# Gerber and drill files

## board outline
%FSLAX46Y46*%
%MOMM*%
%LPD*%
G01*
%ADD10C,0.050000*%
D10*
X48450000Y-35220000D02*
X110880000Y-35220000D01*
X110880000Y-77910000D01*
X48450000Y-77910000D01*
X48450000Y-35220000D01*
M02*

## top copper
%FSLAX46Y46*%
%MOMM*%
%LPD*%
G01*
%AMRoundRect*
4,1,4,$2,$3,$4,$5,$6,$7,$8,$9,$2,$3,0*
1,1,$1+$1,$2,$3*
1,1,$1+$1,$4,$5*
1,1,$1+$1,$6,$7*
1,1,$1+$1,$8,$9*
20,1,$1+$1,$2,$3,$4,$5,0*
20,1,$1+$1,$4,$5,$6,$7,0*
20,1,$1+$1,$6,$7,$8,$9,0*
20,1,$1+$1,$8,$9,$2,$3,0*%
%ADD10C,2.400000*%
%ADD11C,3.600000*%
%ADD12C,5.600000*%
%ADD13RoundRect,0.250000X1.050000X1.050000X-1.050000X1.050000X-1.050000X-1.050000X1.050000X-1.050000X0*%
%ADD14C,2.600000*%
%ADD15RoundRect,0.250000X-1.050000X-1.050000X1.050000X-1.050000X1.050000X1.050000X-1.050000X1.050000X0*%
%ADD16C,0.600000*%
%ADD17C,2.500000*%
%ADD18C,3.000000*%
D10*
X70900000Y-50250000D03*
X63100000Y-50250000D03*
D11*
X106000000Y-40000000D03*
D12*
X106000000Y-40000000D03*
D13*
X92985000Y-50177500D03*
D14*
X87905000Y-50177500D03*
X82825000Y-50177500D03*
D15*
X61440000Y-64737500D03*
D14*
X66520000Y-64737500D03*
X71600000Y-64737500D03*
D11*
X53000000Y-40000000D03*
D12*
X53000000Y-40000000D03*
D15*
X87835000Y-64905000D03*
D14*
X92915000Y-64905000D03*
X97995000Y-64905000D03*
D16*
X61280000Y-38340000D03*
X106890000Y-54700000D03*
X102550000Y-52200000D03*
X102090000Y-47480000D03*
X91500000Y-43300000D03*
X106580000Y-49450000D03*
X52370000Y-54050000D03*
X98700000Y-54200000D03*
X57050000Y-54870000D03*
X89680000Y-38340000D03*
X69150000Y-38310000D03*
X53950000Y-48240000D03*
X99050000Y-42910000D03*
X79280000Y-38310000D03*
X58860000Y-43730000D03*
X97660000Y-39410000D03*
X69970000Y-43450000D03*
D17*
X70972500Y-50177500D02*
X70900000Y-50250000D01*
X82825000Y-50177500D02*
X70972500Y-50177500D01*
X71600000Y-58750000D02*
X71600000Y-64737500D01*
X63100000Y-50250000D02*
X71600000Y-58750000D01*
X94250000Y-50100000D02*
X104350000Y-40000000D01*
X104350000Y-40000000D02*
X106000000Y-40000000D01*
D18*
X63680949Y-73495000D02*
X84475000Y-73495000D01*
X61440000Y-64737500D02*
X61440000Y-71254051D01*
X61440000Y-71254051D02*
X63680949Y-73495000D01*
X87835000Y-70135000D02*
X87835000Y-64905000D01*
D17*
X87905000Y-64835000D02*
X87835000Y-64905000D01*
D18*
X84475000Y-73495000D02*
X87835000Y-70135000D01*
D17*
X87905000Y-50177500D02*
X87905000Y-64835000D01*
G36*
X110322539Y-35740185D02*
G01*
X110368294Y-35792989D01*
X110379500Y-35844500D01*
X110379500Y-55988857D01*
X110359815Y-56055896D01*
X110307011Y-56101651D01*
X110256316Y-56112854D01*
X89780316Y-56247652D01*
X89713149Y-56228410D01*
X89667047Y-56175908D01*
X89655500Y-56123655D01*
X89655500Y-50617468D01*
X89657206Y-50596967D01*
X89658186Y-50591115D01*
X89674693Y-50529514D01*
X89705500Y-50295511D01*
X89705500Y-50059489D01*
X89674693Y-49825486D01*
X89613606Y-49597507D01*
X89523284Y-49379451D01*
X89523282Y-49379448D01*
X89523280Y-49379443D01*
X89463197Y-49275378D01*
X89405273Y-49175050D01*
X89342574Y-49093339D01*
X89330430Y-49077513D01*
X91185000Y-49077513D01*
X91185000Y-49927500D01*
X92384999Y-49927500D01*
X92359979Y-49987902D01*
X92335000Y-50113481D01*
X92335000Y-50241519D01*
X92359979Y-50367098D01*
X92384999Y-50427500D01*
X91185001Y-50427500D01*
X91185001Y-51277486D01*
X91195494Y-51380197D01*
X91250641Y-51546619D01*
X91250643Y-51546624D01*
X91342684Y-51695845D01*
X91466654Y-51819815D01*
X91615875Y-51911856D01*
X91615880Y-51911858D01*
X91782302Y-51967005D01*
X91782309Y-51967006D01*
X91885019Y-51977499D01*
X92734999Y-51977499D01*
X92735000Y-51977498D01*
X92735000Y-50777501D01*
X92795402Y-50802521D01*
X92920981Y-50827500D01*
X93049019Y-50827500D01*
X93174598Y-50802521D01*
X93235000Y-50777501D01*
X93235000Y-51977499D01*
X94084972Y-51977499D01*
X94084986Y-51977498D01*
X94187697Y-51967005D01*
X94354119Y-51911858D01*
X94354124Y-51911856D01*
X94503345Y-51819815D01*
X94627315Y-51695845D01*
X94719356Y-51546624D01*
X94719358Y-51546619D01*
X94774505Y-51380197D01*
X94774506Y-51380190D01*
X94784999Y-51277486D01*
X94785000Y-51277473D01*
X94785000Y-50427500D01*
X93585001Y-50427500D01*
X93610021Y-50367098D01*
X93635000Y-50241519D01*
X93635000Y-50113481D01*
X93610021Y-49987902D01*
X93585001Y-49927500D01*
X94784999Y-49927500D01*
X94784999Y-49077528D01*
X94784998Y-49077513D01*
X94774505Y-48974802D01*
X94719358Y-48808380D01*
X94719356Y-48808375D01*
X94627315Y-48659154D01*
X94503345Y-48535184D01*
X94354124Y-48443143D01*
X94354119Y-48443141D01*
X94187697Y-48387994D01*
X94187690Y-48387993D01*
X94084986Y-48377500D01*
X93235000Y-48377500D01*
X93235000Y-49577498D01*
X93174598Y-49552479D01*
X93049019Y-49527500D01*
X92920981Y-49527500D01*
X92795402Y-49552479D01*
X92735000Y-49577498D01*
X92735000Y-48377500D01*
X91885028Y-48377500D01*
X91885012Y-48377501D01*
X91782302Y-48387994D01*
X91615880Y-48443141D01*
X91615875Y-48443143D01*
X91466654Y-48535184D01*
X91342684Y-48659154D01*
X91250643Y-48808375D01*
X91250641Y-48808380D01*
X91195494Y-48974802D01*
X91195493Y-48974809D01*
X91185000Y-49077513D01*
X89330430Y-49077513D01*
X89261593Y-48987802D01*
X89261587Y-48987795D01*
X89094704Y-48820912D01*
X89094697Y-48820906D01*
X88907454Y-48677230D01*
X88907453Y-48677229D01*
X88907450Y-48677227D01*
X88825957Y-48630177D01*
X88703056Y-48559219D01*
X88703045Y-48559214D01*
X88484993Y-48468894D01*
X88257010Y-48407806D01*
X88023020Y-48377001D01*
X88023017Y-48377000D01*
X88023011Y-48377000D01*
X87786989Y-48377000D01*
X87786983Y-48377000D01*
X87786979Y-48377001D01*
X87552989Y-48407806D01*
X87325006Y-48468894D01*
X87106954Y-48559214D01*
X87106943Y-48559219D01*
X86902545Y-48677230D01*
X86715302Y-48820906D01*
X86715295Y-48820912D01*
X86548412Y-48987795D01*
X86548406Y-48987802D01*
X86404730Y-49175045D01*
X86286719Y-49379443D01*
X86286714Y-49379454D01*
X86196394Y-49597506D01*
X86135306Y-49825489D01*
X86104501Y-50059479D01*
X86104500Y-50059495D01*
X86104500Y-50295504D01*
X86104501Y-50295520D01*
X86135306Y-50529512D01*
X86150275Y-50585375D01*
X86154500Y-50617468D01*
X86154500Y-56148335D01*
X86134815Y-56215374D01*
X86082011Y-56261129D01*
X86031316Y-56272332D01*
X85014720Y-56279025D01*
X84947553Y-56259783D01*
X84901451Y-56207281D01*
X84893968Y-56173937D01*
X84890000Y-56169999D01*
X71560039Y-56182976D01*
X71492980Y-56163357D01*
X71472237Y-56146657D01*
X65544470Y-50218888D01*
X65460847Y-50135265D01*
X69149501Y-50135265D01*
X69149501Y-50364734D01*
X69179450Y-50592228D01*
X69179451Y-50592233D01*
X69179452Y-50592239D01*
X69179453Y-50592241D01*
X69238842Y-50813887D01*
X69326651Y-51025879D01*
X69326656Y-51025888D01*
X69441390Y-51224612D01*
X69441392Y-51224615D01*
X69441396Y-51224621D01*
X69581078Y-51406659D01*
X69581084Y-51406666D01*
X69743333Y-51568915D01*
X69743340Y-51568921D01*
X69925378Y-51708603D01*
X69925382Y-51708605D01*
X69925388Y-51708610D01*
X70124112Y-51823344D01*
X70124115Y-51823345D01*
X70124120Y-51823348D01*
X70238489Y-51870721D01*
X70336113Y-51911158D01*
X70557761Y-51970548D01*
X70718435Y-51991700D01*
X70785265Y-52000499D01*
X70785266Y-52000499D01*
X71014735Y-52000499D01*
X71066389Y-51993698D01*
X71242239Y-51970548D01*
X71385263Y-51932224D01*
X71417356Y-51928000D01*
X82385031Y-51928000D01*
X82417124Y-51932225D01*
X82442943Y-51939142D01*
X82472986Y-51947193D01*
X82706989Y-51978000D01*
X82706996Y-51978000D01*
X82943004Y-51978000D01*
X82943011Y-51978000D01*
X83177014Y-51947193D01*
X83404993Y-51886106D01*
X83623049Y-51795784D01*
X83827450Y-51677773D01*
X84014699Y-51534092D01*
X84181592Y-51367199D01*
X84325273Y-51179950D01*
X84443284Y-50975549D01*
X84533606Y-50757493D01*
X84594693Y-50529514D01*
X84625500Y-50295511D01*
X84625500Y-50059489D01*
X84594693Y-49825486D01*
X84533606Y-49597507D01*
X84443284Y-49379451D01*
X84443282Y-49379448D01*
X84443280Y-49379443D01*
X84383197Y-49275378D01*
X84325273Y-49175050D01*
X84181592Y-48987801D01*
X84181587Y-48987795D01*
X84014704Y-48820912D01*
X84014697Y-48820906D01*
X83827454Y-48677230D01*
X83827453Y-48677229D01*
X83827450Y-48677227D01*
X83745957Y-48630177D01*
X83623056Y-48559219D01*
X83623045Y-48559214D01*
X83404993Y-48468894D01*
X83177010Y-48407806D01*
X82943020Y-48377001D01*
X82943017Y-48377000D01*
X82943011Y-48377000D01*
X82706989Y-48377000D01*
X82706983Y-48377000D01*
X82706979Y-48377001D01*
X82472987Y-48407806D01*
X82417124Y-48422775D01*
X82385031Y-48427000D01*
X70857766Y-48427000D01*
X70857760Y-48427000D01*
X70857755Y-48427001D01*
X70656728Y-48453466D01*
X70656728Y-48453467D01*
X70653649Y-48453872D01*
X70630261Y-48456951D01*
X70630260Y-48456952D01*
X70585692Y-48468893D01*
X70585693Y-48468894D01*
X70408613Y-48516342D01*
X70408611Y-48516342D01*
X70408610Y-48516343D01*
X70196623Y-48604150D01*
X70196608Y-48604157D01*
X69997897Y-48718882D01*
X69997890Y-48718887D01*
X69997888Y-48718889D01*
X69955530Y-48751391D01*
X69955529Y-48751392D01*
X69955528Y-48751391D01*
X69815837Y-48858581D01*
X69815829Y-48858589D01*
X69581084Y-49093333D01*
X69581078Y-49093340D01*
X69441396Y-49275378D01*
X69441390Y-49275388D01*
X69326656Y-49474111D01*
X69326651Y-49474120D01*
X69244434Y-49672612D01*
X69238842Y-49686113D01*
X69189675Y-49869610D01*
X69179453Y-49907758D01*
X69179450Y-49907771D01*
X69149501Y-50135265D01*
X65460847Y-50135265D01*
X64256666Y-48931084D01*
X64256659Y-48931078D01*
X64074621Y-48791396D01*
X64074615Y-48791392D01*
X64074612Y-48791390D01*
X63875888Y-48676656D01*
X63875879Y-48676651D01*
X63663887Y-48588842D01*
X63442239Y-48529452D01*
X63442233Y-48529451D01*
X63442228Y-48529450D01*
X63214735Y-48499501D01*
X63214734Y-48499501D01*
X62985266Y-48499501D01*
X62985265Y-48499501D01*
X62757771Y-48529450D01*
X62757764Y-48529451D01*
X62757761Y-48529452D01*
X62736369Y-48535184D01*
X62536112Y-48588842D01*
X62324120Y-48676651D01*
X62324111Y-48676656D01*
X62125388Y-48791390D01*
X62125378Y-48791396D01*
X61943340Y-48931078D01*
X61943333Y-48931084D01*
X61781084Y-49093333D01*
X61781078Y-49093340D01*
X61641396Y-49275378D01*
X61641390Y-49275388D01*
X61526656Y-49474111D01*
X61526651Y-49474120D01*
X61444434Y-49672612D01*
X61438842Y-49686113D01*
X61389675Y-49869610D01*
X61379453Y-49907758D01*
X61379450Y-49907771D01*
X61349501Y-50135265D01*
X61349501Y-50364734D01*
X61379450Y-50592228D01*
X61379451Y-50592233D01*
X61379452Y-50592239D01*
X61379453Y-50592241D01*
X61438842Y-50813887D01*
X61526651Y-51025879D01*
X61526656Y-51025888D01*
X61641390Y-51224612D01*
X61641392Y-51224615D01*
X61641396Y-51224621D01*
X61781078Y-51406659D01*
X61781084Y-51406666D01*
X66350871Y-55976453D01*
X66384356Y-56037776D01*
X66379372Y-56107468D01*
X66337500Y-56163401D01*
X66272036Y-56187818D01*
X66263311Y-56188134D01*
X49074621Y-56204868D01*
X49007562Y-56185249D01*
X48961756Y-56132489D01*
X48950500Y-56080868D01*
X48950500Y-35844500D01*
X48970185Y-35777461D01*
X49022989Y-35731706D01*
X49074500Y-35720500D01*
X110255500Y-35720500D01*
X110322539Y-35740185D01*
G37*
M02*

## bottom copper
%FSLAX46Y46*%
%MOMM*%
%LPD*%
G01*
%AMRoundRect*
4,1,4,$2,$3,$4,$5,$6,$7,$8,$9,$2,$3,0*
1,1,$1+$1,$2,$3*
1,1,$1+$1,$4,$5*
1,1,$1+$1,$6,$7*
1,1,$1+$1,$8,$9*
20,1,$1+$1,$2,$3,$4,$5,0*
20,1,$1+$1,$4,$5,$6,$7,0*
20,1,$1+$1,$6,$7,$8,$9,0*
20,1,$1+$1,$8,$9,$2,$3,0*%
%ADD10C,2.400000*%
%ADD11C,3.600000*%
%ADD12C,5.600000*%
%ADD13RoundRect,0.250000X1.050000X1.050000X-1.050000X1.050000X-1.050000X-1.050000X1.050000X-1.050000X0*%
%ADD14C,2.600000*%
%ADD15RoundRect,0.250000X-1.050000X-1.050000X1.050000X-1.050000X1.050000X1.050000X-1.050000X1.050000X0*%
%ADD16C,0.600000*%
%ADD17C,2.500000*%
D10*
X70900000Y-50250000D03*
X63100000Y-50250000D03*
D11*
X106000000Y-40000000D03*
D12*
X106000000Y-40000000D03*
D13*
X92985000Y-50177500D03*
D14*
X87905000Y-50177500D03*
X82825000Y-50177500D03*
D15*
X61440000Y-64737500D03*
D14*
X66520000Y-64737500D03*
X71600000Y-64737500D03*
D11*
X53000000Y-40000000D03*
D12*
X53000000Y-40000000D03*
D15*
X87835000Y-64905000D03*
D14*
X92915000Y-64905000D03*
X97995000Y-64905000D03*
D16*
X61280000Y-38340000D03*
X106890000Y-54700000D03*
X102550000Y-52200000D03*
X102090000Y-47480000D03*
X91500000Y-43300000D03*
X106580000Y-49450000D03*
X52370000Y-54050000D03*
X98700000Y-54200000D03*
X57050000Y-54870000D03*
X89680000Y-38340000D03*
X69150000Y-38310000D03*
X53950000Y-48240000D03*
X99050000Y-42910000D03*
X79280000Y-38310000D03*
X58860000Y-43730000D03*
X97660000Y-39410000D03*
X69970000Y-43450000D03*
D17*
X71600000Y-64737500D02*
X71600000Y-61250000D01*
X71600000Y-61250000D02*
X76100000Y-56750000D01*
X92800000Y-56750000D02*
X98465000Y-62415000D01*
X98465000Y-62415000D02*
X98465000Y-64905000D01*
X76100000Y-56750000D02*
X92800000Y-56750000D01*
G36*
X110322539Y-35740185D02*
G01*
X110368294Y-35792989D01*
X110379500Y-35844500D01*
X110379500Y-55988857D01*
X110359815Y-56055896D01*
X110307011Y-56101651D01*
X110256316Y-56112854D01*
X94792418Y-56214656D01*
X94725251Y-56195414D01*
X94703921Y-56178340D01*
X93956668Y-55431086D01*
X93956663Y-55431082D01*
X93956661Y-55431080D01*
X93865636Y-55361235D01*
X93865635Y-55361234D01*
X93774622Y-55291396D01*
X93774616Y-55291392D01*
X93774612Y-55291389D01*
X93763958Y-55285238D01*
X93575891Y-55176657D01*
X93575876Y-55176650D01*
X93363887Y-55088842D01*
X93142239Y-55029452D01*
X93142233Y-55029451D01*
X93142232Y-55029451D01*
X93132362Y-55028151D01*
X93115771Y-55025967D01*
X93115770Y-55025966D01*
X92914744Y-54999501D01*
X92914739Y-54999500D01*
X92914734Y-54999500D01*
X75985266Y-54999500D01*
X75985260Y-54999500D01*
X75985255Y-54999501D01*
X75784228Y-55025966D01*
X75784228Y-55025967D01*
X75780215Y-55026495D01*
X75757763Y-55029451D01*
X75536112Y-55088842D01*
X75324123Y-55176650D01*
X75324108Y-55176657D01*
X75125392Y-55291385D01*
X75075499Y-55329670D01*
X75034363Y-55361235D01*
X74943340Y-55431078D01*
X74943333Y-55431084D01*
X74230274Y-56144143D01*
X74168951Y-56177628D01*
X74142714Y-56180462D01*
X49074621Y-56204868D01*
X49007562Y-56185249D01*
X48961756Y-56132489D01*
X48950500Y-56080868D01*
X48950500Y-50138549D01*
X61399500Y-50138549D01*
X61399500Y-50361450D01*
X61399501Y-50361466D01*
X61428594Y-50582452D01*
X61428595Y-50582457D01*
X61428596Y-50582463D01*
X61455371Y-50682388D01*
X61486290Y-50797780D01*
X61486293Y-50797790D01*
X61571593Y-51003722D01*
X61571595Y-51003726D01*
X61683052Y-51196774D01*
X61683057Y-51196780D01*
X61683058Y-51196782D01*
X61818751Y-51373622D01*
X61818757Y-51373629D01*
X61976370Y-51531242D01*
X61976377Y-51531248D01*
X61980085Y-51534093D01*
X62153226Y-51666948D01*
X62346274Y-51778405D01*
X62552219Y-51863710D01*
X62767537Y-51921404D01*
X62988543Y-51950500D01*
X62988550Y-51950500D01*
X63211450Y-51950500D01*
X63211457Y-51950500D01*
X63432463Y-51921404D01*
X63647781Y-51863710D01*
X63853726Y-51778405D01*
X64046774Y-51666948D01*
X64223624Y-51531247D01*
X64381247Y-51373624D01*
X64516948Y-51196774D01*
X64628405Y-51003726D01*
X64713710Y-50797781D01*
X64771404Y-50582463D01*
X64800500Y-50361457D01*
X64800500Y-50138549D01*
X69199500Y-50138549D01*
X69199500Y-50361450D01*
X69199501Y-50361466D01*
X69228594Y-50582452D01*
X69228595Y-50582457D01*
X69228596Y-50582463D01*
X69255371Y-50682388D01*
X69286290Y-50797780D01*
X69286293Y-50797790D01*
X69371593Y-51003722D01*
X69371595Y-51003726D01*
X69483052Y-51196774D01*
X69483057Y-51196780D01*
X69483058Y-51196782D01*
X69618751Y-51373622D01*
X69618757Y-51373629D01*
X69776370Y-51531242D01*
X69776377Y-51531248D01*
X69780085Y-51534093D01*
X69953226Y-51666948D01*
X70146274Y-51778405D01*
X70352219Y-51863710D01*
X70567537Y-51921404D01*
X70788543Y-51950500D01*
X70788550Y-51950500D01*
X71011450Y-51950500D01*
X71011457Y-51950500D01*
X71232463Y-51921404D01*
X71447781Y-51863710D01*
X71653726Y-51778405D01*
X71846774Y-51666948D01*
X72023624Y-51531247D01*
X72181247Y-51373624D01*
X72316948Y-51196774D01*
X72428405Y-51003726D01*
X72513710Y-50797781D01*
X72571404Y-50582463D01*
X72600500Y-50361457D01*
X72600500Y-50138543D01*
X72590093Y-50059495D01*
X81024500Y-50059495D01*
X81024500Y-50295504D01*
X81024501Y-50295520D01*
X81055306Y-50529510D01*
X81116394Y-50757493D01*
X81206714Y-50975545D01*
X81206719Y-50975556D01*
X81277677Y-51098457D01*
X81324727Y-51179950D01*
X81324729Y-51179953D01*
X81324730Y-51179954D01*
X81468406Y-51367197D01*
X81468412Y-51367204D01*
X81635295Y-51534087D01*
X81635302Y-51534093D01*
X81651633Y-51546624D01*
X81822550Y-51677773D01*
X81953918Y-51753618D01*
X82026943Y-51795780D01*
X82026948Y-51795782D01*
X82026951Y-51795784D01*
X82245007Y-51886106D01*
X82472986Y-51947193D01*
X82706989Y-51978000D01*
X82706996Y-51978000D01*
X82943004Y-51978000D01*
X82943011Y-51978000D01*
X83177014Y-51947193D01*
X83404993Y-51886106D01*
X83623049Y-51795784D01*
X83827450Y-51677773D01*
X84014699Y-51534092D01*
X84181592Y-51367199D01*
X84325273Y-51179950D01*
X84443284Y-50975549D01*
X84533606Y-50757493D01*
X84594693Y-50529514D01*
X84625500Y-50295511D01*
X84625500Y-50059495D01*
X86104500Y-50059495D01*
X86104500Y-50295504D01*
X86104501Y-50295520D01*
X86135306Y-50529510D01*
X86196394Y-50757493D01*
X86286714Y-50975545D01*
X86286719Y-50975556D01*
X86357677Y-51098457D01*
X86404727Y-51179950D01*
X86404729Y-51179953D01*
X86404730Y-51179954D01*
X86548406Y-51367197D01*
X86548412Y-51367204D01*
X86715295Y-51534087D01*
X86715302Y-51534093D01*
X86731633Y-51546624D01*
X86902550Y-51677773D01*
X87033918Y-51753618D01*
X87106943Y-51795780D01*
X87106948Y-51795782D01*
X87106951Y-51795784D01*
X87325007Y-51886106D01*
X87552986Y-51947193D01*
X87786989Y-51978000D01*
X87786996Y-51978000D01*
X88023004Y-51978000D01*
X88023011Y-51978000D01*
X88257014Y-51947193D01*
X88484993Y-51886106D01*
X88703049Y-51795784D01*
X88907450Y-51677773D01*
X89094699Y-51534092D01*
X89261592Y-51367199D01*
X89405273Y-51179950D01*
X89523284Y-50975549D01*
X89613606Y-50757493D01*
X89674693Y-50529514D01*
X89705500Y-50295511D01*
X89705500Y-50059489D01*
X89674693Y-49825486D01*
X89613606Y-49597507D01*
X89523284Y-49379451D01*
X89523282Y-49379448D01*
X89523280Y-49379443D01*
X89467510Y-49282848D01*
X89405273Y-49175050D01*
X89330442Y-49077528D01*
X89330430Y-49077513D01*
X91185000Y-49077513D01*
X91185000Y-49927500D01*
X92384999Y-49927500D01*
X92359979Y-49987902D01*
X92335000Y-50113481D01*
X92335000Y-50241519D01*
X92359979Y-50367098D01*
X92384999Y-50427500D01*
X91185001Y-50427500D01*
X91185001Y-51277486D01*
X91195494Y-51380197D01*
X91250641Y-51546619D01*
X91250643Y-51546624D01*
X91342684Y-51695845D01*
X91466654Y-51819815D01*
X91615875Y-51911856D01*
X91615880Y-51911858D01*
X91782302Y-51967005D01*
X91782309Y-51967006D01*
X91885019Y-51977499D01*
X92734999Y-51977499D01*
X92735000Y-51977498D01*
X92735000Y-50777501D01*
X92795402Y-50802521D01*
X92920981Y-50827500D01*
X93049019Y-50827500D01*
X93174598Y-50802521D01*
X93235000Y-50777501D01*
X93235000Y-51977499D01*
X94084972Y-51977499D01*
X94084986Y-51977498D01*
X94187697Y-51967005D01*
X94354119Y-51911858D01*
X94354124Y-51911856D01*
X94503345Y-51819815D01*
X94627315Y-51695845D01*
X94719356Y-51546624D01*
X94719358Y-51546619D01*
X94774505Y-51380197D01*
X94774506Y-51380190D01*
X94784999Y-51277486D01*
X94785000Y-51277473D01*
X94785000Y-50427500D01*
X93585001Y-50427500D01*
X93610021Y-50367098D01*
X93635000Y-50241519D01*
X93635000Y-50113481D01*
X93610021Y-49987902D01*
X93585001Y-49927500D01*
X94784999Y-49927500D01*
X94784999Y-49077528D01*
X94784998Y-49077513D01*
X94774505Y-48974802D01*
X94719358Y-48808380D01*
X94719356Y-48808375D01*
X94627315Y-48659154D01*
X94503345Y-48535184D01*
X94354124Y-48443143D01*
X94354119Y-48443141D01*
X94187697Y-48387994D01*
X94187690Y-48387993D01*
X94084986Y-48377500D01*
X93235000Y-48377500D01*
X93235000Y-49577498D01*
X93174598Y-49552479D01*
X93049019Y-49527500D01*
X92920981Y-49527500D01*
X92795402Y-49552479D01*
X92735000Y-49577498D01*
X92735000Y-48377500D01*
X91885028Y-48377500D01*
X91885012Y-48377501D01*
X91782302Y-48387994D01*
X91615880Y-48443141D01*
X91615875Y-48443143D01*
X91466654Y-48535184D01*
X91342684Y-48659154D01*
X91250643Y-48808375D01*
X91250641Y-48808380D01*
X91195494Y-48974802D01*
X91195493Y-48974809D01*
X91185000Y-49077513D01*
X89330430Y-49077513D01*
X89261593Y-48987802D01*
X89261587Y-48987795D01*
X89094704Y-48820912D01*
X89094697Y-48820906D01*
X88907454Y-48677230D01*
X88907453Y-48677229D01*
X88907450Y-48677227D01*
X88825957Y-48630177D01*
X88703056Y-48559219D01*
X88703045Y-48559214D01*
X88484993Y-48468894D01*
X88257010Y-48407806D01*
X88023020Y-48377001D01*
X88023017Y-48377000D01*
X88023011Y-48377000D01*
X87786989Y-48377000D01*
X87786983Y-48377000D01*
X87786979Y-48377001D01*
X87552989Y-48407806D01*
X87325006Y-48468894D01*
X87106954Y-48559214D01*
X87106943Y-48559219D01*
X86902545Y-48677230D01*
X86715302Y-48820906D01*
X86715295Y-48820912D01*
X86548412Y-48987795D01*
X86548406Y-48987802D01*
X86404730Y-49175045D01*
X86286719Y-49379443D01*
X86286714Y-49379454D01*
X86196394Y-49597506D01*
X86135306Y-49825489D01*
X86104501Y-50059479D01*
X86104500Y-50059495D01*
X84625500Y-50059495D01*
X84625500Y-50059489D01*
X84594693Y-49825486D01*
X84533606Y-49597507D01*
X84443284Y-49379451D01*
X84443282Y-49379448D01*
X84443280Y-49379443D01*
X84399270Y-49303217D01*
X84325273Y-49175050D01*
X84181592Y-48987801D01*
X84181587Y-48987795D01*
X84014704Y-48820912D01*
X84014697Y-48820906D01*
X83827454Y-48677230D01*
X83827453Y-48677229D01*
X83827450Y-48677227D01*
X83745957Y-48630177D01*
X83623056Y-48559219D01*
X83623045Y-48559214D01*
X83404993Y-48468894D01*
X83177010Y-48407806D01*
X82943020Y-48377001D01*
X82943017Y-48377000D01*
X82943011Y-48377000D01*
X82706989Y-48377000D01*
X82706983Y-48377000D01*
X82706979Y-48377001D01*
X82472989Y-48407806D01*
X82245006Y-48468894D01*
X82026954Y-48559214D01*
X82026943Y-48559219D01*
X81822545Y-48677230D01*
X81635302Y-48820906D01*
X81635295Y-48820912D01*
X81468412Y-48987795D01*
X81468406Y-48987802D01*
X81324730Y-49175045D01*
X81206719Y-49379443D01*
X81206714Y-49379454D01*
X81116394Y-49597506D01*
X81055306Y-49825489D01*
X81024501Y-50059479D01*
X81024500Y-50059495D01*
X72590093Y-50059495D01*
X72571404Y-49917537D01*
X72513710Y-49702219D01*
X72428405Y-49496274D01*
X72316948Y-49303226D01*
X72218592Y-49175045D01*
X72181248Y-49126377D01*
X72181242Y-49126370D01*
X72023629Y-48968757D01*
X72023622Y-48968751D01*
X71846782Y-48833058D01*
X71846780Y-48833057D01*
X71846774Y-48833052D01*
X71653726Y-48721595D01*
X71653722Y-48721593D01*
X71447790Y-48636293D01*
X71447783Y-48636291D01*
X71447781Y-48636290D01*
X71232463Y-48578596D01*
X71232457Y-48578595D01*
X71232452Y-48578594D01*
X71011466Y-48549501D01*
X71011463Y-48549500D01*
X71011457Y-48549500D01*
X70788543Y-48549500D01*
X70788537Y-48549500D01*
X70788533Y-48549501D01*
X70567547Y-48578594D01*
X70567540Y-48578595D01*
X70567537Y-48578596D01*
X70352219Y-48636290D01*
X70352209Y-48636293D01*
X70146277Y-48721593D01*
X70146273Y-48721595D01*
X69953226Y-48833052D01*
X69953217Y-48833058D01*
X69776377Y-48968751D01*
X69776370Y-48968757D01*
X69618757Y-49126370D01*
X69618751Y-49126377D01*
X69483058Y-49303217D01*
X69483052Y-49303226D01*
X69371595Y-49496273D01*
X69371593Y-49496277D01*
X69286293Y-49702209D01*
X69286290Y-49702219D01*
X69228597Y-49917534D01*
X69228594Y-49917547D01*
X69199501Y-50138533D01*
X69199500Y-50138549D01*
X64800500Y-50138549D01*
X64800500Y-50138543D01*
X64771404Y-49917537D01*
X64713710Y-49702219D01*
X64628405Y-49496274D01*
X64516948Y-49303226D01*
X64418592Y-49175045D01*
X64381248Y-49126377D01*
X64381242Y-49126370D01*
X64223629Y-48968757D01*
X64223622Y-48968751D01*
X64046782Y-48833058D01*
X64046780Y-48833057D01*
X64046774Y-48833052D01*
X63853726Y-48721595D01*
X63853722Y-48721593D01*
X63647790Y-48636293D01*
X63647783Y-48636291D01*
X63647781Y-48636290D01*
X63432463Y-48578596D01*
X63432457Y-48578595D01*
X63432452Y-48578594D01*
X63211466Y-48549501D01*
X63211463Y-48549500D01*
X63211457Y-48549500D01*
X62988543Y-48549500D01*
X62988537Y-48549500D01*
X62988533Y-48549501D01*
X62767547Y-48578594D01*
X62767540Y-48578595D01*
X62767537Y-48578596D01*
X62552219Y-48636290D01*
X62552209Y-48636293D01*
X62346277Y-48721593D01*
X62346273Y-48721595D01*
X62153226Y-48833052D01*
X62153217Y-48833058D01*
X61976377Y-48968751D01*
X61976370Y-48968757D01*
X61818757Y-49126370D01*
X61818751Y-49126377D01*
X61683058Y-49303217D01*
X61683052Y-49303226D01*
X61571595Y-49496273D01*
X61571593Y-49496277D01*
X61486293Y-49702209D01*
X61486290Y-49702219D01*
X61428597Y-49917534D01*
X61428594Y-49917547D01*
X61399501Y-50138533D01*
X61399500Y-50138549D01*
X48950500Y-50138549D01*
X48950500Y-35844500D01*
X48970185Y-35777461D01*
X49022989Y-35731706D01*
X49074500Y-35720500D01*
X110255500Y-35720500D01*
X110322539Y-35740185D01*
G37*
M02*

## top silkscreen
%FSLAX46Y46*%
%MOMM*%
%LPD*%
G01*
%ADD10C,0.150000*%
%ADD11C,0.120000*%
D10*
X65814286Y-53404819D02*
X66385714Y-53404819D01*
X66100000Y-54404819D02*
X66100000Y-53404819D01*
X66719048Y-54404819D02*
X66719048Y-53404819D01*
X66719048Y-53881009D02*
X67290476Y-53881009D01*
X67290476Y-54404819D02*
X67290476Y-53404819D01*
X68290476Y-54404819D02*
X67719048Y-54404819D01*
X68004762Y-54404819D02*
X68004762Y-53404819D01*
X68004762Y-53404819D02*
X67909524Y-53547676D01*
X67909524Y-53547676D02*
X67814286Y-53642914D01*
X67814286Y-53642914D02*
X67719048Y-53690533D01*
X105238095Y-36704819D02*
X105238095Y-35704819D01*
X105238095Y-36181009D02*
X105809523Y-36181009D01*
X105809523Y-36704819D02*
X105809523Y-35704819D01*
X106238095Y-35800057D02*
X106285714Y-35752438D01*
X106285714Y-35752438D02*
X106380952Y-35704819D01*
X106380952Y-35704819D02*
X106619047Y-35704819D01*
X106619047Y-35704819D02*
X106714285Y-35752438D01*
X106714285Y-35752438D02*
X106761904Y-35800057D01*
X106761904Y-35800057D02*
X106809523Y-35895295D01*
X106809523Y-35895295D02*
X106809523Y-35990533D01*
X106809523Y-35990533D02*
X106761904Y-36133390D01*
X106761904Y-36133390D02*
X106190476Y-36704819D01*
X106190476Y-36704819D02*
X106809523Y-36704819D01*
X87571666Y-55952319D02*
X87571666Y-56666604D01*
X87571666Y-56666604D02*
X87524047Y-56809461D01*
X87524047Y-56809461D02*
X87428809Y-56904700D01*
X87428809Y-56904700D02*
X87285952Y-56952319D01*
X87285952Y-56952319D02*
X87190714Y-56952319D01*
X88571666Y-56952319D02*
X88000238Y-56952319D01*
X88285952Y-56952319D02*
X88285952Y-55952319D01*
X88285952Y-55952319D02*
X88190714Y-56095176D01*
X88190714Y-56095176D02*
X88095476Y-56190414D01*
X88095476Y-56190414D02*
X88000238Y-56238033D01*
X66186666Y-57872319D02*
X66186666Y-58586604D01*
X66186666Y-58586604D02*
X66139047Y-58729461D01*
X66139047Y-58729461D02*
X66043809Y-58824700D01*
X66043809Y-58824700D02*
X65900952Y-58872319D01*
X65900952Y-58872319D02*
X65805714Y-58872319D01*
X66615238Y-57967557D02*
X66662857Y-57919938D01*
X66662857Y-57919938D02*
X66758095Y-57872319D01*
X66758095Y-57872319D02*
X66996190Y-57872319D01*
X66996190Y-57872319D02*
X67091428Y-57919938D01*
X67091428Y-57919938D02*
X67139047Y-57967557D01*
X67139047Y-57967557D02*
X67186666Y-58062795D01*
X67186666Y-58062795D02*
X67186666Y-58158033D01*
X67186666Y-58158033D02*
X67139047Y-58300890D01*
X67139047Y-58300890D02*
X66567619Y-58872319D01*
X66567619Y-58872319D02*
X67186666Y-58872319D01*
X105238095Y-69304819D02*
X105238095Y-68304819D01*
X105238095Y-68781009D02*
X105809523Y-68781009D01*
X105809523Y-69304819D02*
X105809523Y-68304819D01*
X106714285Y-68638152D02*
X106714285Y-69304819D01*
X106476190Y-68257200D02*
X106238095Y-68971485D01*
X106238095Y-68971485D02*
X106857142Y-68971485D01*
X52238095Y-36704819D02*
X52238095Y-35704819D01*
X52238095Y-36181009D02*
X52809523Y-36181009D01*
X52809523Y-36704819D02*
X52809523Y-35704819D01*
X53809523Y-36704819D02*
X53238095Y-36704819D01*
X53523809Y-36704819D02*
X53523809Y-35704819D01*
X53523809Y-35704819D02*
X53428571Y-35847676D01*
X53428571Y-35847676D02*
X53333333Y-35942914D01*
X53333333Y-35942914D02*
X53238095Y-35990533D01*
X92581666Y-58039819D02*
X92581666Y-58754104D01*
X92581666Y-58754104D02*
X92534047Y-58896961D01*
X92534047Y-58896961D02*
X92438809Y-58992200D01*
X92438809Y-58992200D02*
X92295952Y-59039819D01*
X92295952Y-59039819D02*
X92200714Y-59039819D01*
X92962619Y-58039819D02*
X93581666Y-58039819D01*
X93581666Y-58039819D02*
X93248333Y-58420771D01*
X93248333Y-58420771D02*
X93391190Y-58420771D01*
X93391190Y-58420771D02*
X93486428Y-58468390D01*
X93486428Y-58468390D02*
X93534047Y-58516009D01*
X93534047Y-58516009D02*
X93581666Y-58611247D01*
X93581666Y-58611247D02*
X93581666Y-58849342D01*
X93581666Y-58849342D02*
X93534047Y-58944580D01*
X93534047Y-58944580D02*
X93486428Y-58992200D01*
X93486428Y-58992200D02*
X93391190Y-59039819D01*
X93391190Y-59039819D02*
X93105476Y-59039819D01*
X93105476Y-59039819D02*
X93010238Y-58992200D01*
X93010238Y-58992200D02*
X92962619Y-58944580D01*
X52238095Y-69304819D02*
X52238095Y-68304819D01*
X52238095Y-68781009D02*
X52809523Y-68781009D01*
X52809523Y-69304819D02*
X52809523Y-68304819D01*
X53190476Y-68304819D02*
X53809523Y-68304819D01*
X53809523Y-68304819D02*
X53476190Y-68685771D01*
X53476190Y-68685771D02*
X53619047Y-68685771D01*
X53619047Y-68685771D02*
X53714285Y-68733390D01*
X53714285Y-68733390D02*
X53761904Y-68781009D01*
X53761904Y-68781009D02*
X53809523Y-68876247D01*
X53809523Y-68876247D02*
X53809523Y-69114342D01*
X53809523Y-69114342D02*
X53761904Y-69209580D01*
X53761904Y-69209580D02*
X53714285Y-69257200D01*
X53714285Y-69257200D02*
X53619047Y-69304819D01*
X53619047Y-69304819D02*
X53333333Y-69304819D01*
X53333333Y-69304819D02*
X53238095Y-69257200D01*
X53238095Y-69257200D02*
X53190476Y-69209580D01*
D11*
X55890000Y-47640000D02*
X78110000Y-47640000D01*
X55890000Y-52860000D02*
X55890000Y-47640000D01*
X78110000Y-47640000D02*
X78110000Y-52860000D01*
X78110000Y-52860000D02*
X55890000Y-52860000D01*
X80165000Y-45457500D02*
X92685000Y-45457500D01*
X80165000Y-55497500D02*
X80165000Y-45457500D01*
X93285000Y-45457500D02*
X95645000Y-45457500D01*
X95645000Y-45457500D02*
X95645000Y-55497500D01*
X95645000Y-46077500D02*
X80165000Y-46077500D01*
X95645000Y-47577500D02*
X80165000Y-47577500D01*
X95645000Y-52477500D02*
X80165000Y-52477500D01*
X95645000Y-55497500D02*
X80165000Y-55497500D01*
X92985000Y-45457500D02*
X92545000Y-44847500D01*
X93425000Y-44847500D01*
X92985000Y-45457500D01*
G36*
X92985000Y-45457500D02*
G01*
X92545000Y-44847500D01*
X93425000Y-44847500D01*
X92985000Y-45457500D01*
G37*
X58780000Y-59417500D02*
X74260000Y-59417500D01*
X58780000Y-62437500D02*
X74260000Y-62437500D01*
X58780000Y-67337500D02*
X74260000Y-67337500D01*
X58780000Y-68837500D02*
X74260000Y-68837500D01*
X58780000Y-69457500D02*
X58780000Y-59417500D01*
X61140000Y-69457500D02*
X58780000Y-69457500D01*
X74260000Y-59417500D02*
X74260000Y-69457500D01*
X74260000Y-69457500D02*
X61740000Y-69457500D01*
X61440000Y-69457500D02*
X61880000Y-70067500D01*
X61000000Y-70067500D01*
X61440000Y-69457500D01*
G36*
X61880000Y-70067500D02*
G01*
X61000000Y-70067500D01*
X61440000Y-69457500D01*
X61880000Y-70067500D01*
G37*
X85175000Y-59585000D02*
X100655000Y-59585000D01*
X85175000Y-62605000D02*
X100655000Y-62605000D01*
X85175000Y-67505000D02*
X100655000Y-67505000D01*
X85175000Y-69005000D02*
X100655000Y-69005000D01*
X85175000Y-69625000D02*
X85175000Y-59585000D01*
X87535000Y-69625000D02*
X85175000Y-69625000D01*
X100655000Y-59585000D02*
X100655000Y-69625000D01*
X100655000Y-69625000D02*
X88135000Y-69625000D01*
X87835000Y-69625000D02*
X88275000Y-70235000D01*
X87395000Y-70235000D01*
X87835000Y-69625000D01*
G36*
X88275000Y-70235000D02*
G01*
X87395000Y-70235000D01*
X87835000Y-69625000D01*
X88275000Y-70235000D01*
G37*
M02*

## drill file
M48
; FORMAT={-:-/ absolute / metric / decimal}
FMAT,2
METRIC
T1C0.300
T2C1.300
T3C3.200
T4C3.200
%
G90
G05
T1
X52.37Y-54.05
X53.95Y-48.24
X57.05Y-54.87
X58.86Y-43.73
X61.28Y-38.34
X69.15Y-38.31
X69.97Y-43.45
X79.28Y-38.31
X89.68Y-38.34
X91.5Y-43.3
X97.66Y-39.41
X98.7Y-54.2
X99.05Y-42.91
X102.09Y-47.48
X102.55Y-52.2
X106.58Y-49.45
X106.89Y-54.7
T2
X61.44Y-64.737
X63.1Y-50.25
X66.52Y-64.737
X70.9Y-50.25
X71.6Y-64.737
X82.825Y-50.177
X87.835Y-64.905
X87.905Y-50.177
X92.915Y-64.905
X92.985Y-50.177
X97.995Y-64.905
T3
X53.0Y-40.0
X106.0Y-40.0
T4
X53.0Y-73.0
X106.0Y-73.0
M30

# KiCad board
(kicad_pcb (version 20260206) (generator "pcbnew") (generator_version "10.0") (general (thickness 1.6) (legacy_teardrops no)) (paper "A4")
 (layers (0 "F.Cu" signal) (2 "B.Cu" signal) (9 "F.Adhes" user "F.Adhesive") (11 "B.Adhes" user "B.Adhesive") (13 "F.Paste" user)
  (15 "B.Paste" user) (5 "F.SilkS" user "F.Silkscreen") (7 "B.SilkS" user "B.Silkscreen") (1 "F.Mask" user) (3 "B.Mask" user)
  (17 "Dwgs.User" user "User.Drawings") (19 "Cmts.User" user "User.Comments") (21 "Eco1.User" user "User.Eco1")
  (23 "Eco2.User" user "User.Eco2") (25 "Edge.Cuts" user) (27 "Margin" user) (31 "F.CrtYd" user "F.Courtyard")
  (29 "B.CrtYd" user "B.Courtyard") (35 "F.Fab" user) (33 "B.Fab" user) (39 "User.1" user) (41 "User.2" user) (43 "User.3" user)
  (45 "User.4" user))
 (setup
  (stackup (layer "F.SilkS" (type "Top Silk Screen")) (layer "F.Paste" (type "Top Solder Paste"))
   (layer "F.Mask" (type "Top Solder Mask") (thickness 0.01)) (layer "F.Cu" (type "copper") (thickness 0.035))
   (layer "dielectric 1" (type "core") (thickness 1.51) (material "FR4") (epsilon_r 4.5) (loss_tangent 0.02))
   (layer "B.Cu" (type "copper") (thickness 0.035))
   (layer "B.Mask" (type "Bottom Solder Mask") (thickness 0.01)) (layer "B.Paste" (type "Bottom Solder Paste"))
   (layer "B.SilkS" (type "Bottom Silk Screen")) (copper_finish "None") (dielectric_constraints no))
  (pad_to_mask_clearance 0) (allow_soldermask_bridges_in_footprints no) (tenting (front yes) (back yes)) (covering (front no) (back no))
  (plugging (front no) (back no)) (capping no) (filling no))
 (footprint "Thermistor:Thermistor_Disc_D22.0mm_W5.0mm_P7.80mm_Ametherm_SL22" (layer "F.Cu") (at 70.9 50.25 180)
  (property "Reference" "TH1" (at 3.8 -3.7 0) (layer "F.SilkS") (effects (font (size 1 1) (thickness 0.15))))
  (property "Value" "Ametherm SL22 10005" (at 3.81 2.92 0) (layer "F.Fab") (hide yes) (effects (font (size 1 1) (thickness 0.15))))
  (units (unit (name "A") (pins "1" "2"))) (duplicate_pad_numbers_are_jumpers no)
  (fp_line (start 15.01 2.61) (end -7.21 2.61) (stroke (width 0.12) (type solid)) (layer "F.SilkS"))
  (fp_line (start 15.01 -2.61) (end 15.01 2.61) (stroke (width 0.12) (type solid)) (layer "F.SilkS"))
  (fp_line (start -7.21 2.61) (end -7.21 -2.61) (stroke (width 0.12) (type solid)) (layer "F.SilkS"))
  (fp_line (start -7.21 -2.61) (end 15.01 -2.61) (stroke (width 0.12) (type solid)) (layer "F.SilkS"))
  (pad "1" thru_hole circle (at 0 0 180) (size 2.4 2.4) (drill 1.3) (layers "*.Cu" "*.Mask") (remove_unused_layers no) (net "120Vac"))
  (pad "2" thru_hole circle (at 7.8 0 180) (size 2.4 2.4) (drill 1.3) (layers "*.Cu" "*.Mask") (remove_unused_layers no) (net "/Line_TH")))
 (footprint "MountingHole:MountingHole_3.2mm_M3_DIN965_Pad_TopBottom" (layer "F.Cu") (at 106 40)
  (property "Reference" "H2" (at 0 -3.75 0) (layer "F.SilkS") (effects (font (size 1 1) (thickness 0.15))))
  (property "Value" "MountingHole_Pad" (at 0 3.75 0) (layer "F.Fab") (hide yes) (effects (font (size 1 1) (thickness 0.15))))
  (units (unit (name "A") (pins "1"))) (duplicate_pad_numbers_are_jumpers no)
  (pad "1" thru_hole circle (at 0 0) (size 3.6 3.6) (drill 3.2) (layers "*.Cu" "*.Mask") (remove_unused_layers no) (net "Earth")
   (zone_connect 2))
  (pad "1" connect circle (at 0 0) (size 5.6 5.6) (layers "F.Cu" "F.Mask") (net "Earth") (zone_connect 2))
  (pad "1" connect circle (at 0 0) (size 5.6 5.6) (layers "B.Cu" "B.Mask") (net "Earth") (zone_connect 2)))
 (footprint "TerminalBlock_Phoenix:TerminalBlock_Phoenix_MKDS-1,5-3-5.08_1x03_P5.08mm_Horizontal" (layer "F.Cu") (at 92.985 50.1775 180)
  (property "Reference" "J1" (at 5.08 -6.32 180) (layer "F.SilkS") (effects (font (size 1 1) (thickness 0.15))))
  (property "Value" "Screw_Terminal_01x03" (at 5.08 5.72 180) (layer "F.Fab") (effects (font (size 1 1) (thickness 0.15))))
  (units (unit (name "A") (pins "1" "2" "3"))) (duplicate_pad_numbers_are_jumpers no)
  (fp_line (start 12.82 4.72) (end 0.3 4.72) (stroke (width 0.12) (type solid)) (layer "F.SilkS"))
  (fp_line (start 12.82 -5.32) (end 12.82 4.72) (stroke (width 0.12) (type solid)) (layer "F.SilkS"))
  (fp_line (start -0.3 4.72) (end -2.66 4.72) (stroke (width 0.12) (type solid)) (layer "F.SilkS"))
  (fp_line (start -2.66 4.72) (end -2.66 -5.32) (stroke (width 0.12) (type solid)) (layer "F.SilkS"))
  (fp_line (start -2.66 4.1) (end 12.82 4.1) (stroke (width 0.12) (type solid)) (layer "F.SilkS"))
  (fp_line (start -2.66 2.6) (end 12.82 2.6) (stroke (width 0.12) (type solid)) (layer "F.SilkS"))
  (fp_line (start -2.66 -2.3) (end 12.82 -2.3) (stroke (width 0.12) (type solid)) (layer "F.SilkS"))
  (fp_line (start -2.66 -5.32) (end 12.82 -5.32) (stroke (width 0.12) (type solid)) (layer "F.SilkS"))
  (fp_poly (pts (xy 0 4.72) (xy 0.44 5.33) (xy -0.44 5.33)) (stroke (width 0.12) (type solid)) (fill yes) (layer "F.SilkS"))
  (pad "1" thru_hole roundrect (at 0 0 180) (size 2.6 2.6) (drill 1.3) (layers "*.Cu" "*.Mask") (remove_unused_layers no)
   (roundrect_rratio 0.096154) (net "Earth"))
  (pad "2" thru_hole circle (at 5.08 0 180) (size 2.6 2.6) (drill 1.3) (layers "*.Cu" "*.Mask") (remove_unused_layers no) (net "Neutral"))
  (pad "3" thru_hole circle (at 10.16 0 180) (size 2.6 2.6) (drill 1.3) (layers "*.Cu" "*.Mask") (remove_unused_layers no) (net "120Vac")))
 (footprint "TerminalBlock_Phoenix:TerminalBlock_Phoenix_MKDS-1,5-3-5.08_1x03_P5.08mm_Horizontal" (layer "F.Cu") (at 61.44 64.7375)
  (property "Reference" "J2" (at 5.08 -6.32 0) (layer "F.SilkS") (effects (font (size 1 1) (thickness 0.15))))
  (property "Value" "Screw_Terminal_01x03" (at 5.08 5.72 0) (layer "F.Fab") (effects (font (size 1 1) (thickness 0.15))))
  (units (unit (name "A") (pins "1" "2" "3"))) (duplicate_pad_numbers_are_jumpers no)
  (fp_line (start -2.66 -5.32) (end 12.82 -5.32) (stroke (width 0.12) (type solid)) (layer "F.SilkS"))
  (fp_line (start -2.66 -2.3) (end 12.82 -2.3) (stroke (width 0.12) (type solid)) (layer "F.SilkS"))
  (fp_line (start -2.66 2.6) (end 12.82 2.6) (stroke (width 0.12) (type solid)) (layer "F.SilkS"))
  (fp_line (start -2.66 4.1) (end 12.82 4.1) (stroke (width 0.12) (type solid)) (layer "F.SilkS"))
  (fp_line (start -2.66 4.72) (end -2.66 -5.32) (stroke (width 0.12) (type solid)) (layer "F.SilkS"))
  (fp_line (start -0.3 4.72) (end -2.66 4.72) (stroke (width 0.12) (type solid)) (layer "F.SilkS"))
  (fp_line (start 12.82 -5.32) (end 12.82 4.72) (stroke (width 0.12) (type solid)) (layer "F.SilkS"))
  (fp_line (start 12.82 4.72) (end 0.3 4.72) (stroke (width 0.12) (type solid)) (layer "F.SilkS"))
  (fp_poly (pts (xy 0 4.72) (xy 0.44 5.33) (xy -0.44 5.33)) (stroke (width 0.12) (type solid)) (fill yes) (layer "F.SilkS"))
  (pad "1" thru_hole roundrect (at 0 0) (size 2.6 2.6) (drill 1.3) (layers "*.Cu" "*.Mask") (remove_unused_layers no)
   (roundrect_rratio 0.096154) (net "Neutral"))
  (pad "2" thru_hole circle (at 5.08 0) (size 2.6 2.6) (drill 1.3) (layers "*.Cu" "*.Mask") (remove_unused_layers no)
   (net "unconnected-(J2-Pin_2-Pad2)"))
  (pad "3" thru_hole circle (at 10.16 0) (size 2.6 2.6) (drill 1.3) (layers "*.Cu" "*.Mask") (remove_unused_layers no) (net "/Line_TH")))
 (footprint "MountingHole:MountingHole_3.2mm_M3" (layer "F.Cu") (at 106 73)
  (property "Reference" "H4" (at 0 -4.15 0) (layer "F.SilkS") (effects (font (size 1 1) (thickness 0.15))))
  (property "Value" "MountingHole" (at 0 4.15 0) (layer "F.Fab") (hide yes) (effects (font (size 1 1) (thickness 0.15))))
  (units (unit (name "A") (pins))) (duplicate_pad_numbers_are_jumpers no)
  (pad "" np_thru_hole circle (at 0 0) (size 3.2 3.2) (drill 3.2) (layers "*.Cu" "*.Mask")))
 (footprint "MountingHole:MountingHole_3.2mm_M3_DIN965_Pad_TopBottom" (layer "F.Cu") (at 53 40)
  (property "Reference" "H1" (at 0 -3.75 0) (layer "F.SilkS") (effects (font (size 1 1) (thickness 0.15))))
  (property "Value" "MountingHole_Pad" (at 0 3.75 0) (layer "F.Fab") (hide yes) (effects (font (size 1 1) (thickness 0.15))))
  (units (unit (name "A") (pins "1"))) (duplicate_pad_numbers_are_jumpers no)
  (pad "1" thru_hole circle (at 0 0) (size 3.6 3.6) (drill 3.2) (layers "*.Cu" "*.Mask") (remove_unused_layers no) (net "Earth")
   (zone_connect 2))
  (pad "1" connect circle (at 0 0) (size 5.6 5.6) (layers "F.Cu" "F.Mask") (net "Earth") (zone_connect 2))
  (pad "1" connect circle (at 0 0) (size 5.6 5.6) (layers "B.Cu" "B.Mask") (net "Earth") (zone_connect 2)))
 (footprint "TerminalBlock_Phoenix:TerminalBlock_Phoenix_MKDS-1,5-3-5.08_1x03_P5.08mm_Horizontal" (layer "F.Cu") (at 87.835 64.905)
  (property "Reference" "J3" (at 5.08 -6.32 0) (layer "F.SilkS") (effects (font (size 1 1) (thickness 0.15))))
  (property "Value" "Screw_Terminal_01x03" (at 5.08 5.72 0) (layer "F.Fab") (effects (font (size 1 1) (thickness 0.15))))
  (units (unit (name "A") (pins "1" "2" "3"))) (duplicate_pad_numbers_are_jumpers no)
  (fp_line (start -2.66 -5.32) (end 12.82 -5.32) (stroke (width 0.12) (type solid)) (layer "F.SilkS"))
  (fp_line (start -2.66 -2.3) (end 12.82 -2.3) (stroke (width 0.12) (type solid)) (layer "F.SilkS"))
  (fp_line (start -2.66 2.6) (end 12.82 2.6) (stroke (width 0.12) (type solid)) (layer "F.SilkS"))
  (fp_line (start -2.66 4.1) (end 12.82 4.1) (stroke (width 0.12) (type solid)) (layer "F.SilkS"))
  (fp_line (start -2.66 4.72) (end -2.66 -5.32) (stroke (width 0.12) (type solid)) (layer "F.SilkS"))
  (fp_line (start -0.3 4.72) (end -2.66 4.72) (stroke (width 0.12) (type solid)) (layer "F.SilkS"))
  (fp_line (start 12.82 -5.32) (end 12.82 4.72) (stroke (width 0.12) (type solid)) (layer "F.SilkS"))
  (fp_line (start 12.82 4.72) (end 0.3 4.72) (stroke (width 0.12) (type solid)) (layer "F.SilkS"))
  (fp_poly (pts (xy 0 4.72) (xy 0.44 5.33) (xy -0.44 5.33)) (stroke (width 0.12) (type solid)) (fill yes) (layer "F.SilkS"))
  (pad "1" thru_hole roundrect (at 0 0) (size 2.6 2.6) (drill 1.3) (layers "*.Cu" "*.Mask") (remove_unused_layers no)
   (roundrect_rratio 0.096154) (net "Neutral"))
  (pad "2" thru_hole circle (at 5.08 0) (size 2.6 2.6) (drill 1.3) (layers "*.Cu" "*.Mask") (remove_unused_layers no)
   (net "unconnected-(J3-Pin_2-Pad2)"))
  (pad "3" thru_hole circle (at 10.16 0) (size 2.6 2.6) (drill 1.3) (layers "*.Cu" "*.Mask") (remove_unused_layers no) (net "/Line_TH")))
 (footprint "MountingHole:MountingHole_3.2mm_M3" (layer "F.Cu") (at 53 73)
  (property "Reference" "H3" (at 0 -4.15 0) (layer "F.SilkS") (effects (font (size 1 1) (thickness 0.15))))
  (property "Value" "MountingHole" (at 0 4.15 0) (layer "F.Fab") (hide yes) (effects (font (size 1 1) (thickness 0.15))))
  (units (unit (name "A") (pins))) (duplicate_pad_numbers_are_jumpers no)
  (pad "" np_thru_hole circle (at 0 0) (size 3.2 3.2) (drill 3.2) (layers "*.Cu" "*.Mask")))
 (gr_rect (start 48.45 35.22) (end 110.88 77.91) (stroke (width 0.05) (type default)) (fill no) (layer "Edge.Cuts"))
 (segment (start 70.9725 50.1775) (end 70.9 50.25) (width 2.5) (layer "F.Cu") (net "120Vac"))
 (segment (start 82.825 50.1775) (end 70.9725 50.1775) (width 2.5) (layer "F.Cu") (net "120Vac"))
 (segment (start 71.6 58.75) (end 71.6 64.7375) (width 2.5) (layer "F.Cu") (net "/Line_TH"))
 (segment (start 63.1 50.25) (end 71.6 58.75) (width 2.5) (layer "F.Cu") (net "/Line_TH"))
 (segment (start 71.6 64.7375) (end 71.6 61.25) (width 2.5) (layer "B.Cu") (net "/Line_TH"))
 (segment (start 71.6 61.25) (end 76.1 56.75) (width 2.5) (layer "B.Cu") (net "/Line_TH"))
 (segment (start 92.8 56.75) (end 98.465 62.415) (width 2.5) (layer "B.Cu") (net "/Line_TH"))
 (segment (start 98.465 62.415) (end 98.465 64.905) (width 2.5) (layer "B.Cu") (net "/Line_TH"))
 (segment (start 76.1 56.75) (end 92.8 56.75) (width 2.5) (layer "B.Cu") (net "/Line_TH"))
 (segment (start 94.25 50.1) (end 104.35 40) (width 2.5) (layer "F.Cu") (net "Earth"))
 (segment (start 104.35 40) (end 106 40) (width 2.5) (layer "F.Cu") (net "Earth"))
 (via (at 61.28 38.34) (size 0.6) (drill 0.3) (layers "F.Cu" "B.Cu") (free yes) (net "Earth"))
 (via (at 106.89 54.7) (size 0.6) (drill 0.3) (layers "F.Cu" "B.Cu") (free yes) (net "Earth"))
 (via (at 102.55 52.2) (size 0.6) (drill 0.3) (layers "F.Cu" "B.Cu") (free yes) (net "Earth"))
 (via (at 102.09 47.48) (size 0.6) (drill 0.3) (layers "F.Cu" "B.Cu") (free yes) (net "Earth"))
 (via (at 91.5 43.3) (size 0.6) (drill 0.3) (layers "F.Cu" "B.Cu") (free yes) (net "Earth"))
 (via (at 106.58 49.45) (size 0.6) (drill 0.3) (layers "F.Cu" "B.Cu") (free yes) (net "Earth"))
 (via (at 52.37 54.05) (size 0.6) (drill 0.3) (layers "F.Cu" "B.Cu") (free yes) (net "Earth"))
 (via (at 98.7 54.2) (size 0.6) (drill 0.3) (layers "F.Cu" "B.Cu") (free yes) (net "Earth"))
 (via (at 57.05 54.87) (size 0.6) (drill 0.3) (layers "F.Cu" "B.Cu") (free yes) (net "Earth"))
 (via (at 89.68 38.34) (size 0.6) (drill 0.3) (layers "F.Cu" "B.Cu") (free yes) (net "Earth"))
 (via (at 69.15 38.31) (size 0.6) (drill 0.3) (layers "F.Cu" "B.Cu") (free yes) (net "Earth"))
 (via (at 53.95 48.24) (size 0.6) (drill 0.3) (layers "F.Cu" "B.Cu") (free yes) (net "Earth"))
 (via (at 99.05 42.91) (size 0.6) (drill 0.3) (layers "F.Cu" "B.Cu") (free yes) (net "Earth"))
 (via (at 79.28 38.31) (size 0.6) (drill 0.3) (layers "F.Cu" "B.Cu") (free yes) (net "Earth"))
 (via (at 58.86 43.73) (size 0.6) (drill 0.3) (layers "F.Cu" "B.Cu") (free yes) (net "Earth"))
 (via (at 97.66 39.41) (size 0.6) (drill 0.3) (layers "F.Cu" "B.Cu") (free yes) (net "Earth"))
 (via (at 69.97 43.45) (size 0.6) (drill 0.3) (layers "F.Cu" "B.Cu") (free yes) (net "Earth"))
 (segment (start 63.680949 73.495) (end 84.475 73.495) (width 3) (layer "F.Cu") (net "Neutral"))
 (segment (start 61.44 64.7375) (end 61.44 71.254051) (width 3) (layer "F.Cu") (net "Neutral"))
 (segment (start 61.44 71.254051) (end 63.680949 73.495) (width 3) (layer "F.Cu") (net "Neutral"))
 (segment (start 87.835 70.135) (end 87.835 64.905) (width 3) (layer "F.Cu") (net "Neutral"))
 (segment (start 87.905 64.835) (end 87.835 64.905) (width 2.5) (layer "F.Cu") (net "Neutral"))
 (segment (start 84.475 73.495) (end 87.835 70.135) (width 3) (layer "F.Cu") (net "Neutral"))
 (segment (start 87.905 50.1775) (end 87.905 64.835) (width 2.5) (layer "F.Cu") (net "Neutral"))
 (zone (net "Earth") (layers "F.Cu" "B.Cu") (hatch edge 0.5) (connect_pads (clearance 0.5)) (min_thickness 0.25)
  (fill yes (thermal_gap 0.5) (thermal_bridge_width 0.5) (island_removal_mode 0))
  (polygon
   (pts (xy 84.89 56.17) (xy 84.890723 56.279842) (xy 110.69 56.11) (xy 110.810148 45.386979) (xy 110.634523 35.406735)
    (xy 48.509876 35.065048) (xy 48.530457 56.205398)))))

